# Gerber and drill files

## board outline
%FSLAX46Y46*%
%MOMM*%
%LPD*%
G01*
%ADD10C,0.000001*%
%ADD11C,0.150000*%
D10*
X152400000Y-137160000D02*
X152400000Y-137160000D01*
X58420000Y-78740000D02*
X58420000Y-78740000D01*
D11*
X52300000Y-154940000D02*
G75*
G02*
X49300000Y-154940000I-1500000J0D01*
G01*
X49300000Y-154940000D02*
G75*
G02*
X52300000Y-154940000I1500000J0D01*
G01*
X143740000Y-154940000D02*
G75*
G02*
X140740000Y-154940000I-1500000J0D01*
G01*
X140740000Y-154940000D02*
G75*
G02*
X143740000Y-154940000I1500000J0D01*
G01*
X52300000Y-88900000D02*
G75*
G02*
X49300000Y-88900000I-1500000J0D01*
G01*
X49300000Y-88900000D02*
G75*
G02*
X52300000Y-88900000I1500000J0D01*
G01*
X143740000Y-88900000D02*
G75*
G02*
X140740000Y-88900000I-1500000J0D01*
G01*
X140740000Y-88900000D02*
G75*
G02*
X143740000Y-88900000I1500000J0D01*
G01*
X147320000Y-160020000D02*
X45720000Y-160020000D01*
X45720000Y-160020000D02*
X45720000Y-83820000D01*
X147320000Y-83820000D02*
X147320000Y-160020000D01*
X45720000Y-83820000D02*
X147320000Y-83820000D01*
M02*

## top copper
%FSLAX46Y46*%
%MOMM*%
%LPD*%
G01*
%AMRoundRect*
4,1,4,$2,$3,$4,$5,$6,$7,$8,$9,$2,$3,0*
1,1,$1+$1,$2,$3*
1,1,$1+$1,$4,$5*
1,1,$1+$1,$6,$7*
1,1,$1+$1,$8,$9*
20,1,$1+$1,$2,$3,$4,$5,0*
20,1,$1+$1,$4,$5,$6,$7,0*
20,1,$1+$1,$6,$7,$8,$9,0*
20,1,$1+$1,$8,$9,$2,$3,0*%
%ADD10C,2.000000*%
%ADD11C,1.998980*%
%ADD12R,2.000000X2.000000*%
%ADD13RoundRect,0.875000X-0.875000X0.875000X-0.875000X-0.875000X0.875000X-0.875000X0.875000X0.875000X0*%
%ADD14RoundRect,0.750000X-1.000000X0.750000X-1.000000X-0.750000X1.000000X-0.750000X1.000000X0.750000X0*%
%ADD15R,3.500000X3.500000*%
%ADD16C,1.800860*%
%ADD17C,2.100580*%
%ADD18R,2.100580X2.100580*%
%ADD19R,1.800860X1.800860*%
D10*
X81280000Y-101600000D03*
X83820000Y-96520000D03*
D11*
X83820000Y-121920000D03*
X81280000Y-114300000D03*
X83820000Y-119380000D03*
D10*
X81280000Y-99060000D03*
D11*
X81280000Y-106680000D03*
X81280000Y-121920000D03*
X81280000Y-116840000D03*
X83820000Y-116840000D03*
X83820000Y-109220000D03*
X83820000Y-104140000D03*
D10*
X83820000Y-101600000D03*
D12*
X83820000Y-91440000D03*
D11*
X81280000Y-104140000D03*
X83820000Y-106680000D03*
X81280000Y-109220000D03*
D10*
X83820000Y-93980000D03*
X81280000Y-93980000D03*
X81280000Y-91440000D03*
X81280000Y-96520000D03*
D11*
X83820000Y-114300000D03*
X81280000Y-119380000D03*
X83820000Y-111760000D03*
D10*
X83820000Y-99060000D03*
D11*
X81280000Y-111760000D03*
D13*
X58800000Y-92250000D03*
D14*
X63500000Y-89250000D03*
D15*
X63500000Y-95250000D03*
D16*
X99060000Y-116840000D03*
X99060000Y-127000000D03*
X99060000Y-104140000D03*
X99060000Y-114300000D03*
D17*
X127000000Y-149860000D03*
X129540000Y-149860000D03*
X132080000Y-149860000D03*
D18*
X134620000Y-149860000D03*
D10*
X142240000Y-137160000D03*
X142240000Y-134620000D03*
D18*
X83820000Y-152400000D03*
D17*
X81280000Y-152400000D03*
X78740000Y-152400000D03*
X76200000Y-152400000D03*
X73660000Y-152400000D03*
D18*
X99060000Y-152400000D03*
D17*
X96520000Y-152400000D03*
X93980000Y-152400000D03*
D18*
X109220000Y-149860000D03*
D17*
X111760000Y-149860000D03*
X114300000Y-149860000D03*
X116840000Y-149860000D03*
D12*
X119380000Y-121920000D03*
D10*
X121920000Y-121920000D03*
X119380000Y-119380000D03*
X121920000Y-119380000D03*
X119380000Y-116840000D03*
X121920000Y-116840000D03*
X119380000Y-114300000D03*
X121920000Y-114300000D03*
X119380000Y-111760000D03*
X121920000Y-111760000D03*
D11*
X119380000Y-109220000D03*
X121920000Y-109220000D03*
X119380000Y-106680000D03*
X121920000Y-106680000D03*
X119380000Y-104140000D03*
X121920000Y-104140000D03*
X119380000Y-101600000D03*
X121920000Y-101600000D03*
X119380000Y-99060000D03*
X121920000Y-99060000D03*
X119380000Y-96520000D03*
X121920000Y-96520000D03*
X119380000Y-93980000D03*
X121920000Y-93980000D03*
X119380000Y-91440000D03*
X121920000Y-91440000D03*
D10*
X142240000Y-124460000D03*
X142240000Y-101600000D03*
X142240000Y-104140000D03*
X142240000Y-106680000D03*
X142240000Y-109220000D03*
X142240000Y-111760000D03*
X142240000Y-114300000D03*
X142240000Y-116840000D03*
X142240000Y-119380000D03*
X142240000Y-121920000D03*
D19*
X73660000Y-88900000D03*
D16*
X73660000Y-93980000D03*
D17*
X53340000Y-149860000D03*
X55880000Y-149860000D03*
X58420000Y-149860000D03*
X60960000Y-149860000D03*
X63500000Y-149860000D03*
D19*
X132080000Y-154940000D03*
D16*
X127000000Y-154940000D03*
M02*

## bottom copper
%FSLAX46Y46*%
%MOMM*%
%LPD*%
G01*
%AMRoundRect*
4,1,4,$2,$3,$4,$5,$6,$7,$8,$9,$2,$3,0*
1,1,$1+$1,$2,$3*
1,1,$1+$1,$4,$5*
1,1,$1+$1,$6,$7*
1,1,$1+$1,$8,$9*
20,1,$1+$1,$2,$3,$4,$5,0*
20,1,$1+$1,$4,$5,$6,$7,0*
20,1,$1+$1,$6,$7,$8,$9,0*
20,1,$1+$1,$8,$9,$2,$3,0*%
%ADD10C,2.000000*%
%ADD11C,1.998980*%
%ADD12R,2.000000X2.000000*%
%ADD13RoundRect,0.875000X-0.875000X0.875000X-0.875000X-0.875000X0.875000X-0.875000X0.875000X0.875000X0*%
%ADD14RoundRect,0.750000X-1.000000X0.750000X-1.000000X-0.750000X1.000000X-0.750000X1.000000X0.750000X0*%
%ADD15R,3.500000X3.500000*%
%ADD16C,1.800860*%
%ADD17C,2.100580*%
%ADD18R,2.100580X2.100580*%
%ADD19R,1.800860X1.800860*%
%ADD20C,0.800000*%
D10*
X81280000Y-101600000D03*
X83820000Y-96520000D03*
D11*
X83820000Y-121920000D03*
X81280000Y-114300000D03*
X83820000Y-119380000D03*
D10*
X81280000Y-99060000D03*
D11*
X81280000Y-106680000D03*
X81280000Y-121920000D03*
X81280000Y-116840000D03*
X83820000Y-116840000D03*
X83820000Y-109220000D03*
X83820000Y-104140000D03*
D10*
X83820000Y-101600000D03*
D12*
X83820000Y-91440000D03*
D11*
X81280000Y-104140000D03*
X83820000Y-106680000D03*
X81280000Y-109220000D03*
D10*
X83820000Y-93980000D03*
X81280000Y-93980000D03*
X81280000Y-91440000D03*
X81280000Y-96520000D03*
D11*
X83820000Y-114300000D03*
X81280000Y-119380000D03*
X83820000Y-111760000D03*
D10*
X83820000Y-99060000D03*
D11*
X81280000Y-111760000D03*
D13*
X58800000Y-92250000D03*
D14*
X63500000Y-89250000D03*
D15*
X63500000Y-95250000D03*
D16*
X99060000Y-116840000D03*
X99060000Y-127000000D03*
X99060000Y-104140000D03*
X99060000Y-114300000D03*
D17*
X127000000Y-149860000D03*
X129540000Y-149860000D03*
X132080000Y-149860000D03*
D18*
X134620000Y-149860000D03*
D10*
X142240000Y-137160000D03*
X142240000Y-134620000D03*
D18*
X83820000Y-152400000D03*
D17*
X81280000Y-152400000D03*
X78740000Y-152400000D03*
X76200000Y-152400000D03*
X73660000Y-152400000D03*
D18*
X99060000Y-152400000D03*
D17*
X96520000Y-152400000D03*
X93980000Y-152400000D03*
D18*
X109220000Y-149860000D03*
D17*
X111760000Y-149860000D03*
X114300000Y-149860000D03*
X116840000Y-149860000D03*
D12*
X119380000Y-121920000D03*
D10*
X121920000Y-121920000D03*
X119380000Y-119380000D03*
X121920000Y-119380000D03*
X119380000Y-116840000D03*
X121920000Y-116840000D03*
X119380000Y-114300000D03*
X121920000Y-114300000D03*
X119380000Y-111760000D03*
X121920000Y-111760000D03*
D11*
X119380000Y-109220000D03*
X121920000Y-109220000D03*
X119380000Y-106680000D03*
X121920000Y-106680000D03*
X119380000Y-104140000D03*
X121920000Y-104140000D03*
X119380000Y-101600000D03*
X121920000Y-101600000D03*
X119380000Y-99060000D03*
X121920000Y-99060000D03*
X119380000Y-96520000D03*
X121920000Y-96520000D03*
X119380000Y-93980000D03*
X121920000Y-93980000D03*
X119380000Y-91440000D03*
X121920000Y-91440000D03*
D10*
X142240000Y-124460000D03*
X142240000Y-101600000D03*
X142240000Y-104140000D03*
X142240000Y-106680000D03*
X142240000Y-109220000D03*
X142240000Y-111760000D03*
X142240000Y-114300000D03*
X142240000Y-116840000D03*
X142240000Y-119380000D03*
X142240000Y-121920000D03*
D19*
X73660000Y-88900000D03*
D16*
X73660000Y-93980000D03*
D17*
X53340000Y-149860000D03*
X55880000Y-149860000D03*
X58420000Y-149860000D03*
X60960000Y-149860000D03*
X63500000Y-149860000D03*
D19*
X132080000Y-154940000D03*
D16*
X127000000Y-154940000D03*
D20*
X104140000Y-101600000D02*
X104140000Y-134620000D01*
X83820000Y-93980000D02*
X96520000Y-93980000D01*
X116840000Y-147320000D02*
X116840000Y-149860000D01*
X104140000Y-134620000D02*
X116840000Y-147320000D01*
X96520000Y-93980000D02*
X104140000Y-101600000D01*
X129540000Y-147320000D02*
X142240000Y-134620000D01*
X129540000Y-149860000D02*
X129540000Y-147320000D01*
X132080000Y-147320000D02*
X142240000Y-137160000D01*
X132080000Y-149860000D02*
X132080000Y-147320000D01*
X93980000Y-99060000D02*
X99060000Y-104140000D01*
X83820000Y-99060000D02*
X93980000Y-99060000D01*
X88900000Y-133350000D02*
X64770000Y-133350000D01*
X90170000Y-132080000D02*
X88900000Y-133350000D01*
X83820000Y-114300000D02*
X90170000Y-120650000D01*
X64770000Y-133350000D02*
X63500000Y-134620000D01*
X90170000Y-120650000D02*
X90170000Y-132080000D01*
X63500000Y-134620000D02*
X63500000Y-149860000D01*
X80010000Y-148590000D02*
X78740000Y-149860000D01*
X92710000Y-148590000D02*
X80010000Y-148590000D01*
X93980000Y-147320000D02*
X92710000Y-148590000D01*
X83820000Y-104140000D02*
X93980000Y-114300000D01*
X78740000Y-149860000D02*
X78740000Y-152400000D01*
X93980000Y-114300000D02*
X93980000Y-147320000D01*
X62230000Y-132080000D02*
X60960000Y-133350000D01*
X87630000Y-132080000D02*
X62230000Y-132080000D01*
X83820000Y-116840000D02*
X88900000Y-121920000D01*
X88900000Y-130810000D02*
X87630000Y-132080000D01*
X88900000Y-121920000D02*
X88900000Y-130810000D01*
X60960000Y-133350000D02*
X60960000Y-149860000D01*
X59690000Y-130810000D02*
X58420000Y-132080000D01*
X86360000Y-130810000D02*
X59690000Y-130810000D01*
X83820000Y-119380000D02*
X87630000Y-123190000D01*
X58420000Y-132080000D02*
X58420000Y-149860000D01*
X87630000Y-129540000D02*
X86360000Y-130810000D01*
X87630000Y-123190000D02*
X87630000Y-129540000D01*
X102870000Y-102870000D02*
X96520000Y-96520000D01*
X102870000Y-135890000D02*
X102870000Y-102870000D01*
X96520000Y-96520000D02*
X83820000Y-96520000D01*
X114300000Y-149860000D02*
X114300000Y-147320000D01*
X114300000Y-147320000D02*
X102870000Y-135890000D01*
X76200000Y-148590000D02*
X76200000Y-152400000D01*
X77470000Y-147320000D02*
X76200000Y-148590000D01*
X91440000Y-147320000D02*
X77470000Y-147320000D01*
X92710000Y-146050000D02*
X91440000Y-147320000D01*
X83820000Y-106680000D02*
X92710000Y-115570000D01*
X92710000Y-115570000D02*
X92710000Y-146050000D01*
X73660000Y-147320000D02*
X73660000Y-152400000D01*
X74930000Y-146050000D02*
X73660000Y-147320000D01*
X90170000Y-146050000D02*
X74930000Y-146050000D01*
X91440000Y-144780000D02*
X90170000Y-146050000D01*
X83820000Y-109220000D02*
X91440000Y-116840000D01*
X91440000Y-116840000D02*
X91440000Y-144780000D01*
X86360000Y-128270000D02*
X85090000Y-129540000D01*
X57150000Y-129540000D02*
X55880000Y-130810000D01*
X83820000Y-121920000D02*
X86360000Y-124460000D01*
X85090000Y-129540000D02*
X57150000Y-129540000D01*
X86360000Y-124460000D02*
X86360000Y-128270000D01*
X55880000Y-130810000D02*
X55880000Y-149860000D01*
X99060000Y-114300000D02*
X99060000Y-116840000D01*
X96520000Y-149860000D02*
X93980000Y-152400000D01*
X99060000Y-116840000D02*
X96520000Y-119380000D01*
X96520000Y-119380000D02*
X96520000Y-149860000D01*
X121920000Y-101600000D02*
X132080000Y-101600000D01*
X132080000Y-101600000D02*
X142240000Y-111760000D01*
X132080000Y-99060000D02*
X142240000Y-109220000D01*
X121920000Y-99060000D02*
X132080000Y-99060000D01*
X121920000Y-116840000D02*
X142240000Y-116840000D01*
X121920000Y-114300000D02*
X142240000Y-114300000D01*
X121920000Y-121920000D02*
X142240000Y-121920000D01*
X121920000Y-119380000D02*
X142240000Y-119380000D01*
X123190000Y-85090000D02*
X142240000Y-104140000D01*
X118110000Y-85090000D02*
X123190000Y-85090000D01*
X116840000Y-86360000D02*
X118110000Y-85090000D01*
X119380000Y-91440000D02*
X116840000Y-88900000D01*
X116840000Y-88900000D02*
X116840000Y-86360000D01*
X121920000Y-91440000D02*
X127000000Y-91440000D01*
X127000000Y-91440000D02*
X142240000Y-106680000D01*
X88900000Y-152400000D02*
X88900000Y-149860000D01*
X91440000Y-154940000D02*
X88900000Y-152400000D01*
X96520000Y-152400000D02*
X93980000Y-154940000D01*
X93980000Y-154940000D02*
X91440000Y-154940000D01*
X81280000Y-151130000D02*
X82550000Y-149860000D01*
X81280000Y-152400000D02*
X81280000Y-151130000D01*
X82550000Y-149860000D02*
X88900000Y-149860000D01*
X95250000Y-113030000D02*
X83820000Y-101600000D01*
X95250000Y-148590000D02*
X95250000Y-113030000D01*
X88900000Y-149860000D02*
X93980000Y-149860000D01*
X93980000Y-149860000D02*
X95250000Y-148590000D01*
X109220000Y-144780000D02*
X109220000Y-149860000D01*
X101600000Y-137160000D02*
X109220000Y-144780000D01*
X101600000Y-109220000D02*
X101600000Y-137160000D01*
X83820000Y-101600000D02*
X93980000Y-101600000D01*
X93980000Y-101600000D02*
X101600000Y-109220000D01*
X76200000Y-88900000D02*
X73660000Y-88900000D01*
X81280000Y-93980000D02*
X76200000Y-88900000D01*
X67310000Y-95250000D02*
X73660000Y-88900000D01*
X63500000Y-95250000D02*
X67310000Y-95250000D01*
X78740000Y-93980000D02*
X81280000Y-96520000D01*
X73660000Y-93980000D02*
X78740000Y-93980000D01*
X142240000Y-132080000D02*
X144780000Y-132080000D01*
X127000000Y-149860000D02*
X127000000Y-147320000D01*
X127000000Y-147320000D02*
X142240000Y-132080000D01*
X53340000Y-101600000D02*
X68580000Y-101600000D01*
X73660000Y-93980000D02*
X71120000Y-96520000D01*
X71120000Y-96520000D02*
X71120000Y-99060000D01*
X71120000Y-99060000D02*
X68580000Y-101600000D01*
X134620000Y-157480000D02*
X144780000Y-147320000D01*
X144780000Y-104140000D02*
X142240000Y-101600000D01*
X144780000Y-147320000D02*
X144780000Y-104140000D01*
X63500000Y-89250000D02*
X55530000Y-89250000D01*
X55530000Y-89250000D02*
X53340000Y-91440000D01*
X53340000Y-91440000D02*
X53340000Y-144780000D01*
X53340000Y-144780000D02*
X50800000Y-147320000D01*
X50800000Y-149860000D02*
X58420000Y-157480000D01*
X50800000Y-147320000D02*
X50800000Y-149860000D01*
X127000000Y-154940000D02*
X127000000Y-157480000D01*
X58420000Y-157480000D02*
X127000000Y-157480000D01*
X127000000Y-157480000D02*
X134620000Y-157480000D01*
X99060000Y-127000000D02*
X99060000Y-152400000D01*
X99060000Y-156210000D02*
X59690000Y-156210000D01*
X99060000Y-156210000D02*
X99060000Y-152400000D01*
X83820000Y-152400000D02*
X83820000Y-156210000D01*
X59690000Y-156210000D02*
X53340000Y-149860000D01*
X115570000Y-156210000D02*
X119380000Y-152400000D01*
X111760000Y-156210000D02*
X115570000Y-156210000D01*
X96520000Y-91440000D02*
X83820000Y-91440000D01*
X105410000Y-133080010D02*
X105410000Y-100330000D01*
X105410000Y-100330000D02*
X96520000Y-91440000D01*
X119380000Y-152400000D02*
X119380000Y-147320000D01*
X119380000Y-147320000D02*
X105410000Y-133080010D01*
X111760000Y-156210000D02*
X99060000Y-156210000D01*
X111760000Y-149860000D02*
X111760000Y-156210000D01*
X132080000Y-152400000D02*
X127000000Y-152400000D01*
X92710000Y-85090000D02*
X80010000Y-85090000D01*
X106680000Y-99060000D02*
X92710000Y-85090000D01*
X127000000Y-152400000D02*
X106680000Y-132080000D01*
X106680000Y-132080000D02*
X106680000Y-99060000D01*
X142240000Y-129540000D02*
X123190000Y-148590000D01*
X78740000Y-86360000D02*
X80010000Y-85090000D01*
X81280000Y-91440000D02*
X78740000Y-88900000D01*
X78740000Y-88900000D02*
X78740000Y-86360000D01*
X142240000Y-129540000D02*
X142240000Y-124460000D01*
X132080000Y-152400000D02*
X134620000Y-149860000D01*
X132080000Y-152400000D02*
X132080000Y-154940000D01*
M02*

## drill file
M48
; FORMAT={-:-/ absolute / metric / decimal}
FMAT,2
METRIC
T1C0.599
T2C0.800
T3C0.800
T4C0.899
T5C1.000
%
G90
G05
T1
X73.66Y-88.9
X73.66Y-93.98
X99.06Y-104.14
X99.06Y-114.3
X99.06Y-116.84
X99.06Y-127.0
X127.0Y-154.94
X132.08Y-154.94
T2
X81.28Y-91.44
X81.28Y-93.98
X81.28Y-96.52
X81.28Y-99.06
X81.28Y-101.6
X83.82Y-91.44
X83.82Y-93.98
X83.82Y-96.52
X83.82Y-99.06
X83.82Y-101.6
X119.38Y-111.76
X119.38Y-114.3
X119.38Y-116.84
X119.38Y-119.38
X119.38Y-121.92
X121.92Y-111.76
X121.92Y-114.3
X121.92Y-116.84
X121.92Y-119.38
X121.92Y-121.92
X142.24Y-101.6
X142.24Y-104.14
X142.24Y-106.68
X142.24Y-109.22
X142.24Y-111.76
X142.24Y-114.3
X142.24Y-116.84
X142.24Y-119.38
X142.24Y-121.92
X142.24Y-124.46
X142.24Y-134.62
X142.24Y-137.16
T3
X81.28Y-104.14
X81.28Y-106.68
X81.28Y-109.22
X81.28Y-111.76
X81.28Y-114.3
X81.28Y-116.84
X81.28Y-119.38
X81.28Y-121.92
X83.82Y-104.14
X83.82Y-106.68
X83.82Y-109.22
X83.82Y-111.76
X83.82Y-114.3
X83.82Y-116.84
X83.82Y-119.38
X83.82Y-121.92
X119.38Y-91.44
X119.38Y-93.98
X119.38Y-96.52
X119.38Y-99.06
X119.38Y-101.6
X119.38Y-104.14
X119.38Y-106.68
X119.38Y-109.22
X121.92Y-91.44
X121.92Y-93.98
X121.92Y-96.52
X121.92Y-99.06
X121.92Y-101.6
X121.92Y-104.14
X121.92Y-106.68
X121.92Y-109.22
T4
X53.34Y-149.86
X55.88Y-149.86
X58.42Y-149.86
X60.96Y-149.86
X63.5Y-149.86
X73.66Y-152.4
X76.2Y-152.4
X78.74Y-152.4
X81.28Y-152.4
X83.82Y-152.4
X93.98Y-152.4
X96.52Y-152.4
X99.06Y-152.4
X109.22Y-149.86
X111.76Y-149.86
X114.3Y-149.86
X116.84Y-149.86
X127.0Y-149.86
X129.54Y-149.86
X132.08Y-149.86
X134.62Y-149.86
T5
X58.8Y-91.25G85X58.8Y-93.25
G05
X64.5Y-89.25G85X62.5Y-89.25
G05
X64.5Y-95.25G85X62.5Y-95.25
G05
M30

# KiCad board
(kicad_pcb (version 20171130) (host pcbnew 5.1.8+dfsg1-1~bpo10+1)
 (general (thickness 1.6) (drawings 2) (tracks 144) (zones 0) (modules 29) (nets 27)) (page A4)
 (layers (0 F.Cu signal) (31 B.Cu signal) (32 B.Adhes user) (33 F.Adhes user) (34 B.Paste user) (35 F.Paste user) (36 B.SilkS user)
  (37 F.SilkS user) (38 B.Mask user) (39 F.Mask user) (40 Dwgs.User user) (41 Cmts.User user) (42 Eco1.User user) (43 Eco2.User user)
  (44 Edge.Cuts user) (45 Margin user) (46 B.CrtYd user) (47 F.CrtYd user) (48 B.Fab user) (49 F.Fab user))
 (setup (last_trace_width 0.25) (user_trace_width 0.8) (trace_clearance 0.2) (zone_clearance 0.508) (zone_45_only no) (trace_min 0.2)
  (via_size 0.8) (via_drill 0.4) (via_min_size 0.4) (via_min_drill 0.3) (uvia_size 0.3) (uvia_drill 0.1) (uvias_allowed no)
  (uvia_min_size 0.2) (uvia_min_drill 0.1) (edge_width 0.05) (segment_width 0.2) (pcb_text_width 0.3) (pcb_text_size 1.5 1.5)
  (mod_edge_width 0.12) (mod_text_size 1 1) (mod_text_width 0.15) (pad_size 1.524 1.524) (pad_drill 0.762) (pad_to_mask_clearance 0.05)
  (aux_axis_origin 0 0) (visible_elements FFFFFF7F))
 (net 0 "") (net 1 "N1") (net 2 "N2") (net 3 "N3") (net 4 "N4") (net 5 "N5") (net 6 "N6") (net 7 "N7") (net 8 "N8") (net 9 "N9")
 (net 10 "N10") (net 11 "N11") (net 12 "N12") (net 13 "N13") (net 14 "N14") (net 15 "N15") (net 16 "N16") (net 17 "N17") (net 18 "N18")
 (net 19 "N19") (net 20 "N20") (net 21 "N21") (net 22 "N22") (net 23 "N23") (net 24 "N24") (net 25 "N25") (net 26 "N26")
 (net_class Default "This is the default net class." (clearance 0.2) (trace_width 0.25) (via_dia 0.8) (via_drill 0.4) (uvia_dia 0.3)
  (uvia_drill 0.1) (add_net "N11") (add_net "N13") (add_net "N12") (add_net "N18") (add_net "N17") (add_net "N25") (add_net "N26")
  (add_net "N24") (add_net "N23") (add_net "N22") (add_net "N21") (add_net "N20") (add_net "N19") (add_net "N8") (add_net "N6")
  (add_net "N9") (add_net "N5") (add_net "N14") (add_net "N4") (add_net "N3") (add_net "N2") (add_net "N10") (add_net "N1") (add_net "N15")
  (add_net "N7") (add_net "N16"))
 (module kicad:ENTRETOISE (layer F.Cu) (at 50.8 154.94)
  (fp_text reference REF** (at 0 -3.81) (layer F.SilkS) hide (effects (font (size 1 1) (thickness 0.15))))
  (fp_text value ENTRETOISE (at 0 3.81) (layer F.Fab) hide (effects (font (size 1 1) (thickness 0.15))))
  (fp_circle (center 0 0) (end 1.5 0) (layer Edge.Cuts) (width 0.15)))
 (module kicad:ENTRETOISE (layer F.Cu) (at 142.24 154.94)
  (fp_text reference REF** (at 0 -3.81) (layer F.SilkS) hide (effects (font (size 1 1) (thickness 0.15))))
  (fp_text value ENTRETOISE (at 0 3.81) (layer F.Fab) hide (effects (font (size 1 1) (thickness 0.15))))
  (fp_circle (center 0 0) (end 1.5 0) (layer Edge.Cuts) (width 0.15)))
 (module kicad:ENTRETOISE (layer F.Cu) (at 50.8 88.9)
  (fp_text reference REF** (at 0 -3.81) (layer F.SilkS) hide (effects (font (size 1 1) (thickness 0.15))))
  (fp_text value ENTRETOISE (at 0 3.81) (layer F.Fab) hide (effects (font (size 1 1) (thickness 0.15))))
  (fp_circle (center 0 0) (end 1.5 0) (layer Edge.Cuts) (width 0.15)))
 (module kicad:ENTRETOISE (layer F.Cu) (at 142.24 88.9)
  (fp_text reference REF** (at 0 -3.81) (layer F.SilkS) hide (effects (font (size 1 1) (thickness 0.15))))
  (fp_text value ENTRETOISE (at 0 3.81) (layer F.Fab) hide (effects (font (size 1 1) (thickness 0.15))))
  (fp_circle (center 0 0) (end 1.5 0) (layer Edge.Cuts) (width 0.15)))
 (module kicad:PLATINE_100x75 (layer F.Cu) (at 96.52 121.92)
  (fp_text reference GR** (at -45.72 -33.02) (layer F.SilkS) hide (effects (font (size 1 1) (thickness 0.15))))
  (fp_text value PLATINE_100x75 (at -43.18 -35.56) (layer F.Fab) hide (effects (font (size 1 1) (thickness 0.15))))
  (fp_line (start 50.8 38.1) (end -50.8 38.1) (layer Edge.Cuts) (width 0.15))
  (fp_line (start -50.8 38.1) (end -50.8 -38.1) (layer Edge.Cuts) (width 0.15))
  (fp_line (start 50.8 -38.1) (end 50.8 38.1) (layer Edge.Cuts) (width 0.15))
  (fp_line (start -50.8 -38.1) (end 50.8 -38.1) (layer Edge.Cuts) (width 0.15)))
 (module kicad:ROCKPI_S (layer F.Cu) (at 101.6 106.68)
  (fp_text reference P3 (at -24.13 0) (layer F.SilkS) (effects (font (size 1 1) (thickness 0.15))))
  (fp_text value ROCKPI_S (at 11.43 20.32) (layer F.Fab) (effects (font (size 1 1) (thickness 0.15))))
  (pad 10 thru_hole circle (at -20.32 -5.08 270) (size 2 2) (drill 0.8) (layers *.Cu *.Mask F.SilkS))
  (pad 5 thru_hole circle (at -17.78 -10.16 270) (size 2 2) (drill 0.8) (layers *.Cu *.Mask F.SilkS) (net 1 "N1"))
  (pad 25 thru_hole circle (at -17.78 15.24 270) (size 1.99898 1.99898) (drill 0.8001) (layers *.Cu *.Mask F.SilkS) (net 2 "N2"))
  (pad 20 thru_hole circle (at -20.32 7.62 270) (size 1.99898 1.99898) (drill 0.8001) (layers *.Cu *.Mask F.SilkS))
  (pad 23 thru_hole circle (at -17.78 12.7 270) (size 1.99898 1.99898) (drill 0.8001) (layers *.Cu *.Mask F.SilkS) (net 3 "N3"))
  (pad 8 thru_hole circle (at -20.32 -7.62 270) (size 2 2) (drill 0.8) (layers *.Cu *.Mask F.SilkS))
  (pad 14 thru_hole circle (at -20.32 0 270) (size 1.99898 1.99898) (drill 0.8001) (layers *.Cu *.Mask F.SilkS))
  (pad 26 thru_hole circle (at -20.32 15.24 270) (size 1.99898 1.99898) (drill 0.8001) (layers *.Cu *.Mask F.SilkS))
  (pad 22 thru_hole circle (at -20.32 10.16 270) (size 1.99898 1.99898) (drill 0.8001) (layers *.Cu *.Mask F.SilkS))
  (pad 21 thru_hole circle (at -17.78 10.16 270) (size 1.99898 1.99898) (drill 0.8001) (layers *.Cu *.Mask F.SilkS) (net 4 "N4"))
  (pad 15 thru_hole circle (at -17.78 2.54 270) (size 1.99898 1.99898) (drill 0.8001) (layers *.Cu *.Mask F.SilkS) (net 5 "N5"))
  (pad 11 thru_hole circle (at -17.78 -2.54 270) (size 1.99898 1.99898) (drill 0.8001) (layers *.Cu *.Mask F.SilkS) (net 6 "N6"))
  (pad 9 thru_hole circle (at -17.78 -5.08 270) (size 2 2) (drill 0.8) (layers *.Cu *.Mask F.SilkS) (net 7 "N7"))
  (pad 1 thru_hole rect (at -17.78 -15.24 270) (size 2 2) (drill 0.8) (layers *.Cu *.Mask F.SilkS) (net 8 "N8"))
  (pad 12 thru_hole circle (at -20.32 -2.54 270) (size 1.99898 1.99898) (drill 0.8001) (layers *.Cu *.Mask F.SilkS))
  (pad 13 thru_hole circle (at -17.78 0 270) (size 1.99898 1.99898) (drill 0.8001) (layers *.Cu *.Mask F.SilkS) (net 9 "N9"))
  (pad 16 thru_hole circle (at -20.32 2.54 270) (size 1.99898 1.99898) (drill 0.8001) (layers *.Cu *.Mask F.SilkS))
  (pad 3 thru_hole circle (at -17.78 -12.7 270) (size 2 2) (drill 0.8) (layers *.Cu *.Mask F.SilkS) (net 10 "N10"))
  (pad 4 thru_hole circle (at -20.32 -12.7 270) (size 2 2) (drill 0.8) (layers *.Cu *.Mask F.SilkS) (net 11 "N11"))
  (pad 2 thru_hole circle (at -20.32 -15.24 270) (size 2 2) (drill 0.8) (layers *.Cu *.Mask F.SilkS) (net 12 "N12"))
  (pad 6 thru_hole circle (at -20.32 -10.16 270) (size 2 2) (drill 0.8) (layers *.Cu *.Mask F.SilkS) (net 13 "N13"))
  (pad 19 thru_hole circle (at -17.78 7.62 270) (size 1.99898 1.99898) (drill 0.8001) (layers *.Cu *.Mask F.SilkS) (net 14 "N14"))
  (pad 24 thru_hole circle (at -20.32 12.7 270) (size 1.99898 1.99898) (drill 0.8001) (layers *.Cu *.Mask F.SilkS))
  (pad 17 thru_hole circle (at -17.78 5.08) (size 1.99898 1.99898) (drill 0.8001) (layers *.Cu *.Mask F.SilkS))
  (pad 7 thru_hole circle (at -17.78 -7.62 270) (size 2 2) (drill 0.8) (layers *.Cu *.Mask F.SilkS) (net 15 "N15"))
  (pad 18 thru_hole circle (at -20.32 5.08 270) (size 1.99898 1.99898) (drill 0.8001) (layers *.Cu *.Mask F.SilkS)))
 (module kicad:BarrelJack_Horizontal (layer F.Cu) (at 63.5 95.25 270)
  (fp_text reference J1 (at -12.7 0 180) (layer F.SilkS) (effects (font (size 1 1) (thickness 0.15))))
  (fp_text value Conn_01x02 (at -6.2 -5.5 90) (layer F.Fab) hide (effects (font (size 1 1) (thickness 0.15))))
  (pad 3 thru_hole roundrect (at -3 4.7 270) (size 3.5 3.5) (drill oval 3 1) (layers *.Cu *.Mask) (roundrect_rratio 0.25))
  (pad 2 thru_hole roundrect (at -6 0 270) (size 3 3.5) (drill oval 1 3) (layers *.Cu *.Mask) (roundrect_rratio 0.25) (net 13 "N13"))
  (pad 1 thru_hole rect (at 0 0 270) (size 3.5 3.5) (drill oval 1 3) (layers *.Cu *.Mask) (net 11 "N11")))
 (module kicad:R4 (layer F.Cu) (at 99.06 121.92 270) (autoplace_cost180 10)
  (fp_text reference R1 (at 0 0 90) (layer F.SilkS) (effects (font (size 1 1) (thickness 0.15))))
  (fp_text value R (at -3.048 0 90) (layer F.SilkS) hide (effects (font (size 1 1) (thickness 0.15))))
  (pad 1 thru_hole circle (at -5.08 0 270) (size 1.80086 1.80086) (drill 0.59944) (layers *.Cu *.Mask F.SilkS) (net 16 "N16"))
  (pad 2 thru_hole circle (at 5.08 0 270) (size 1.80086 1.80086) (drill 0.59944) (layers *.Cu *.Mask F.SilkS) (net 8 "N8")))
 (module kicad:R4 (layer F.Cu) (at 99.06 109.22 270) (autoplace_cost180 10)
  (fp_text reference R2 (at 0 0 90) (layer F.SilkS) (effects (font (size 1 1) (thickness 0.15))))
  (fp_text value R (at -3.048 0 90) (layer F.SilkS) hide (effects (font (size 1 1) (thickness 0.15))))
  (pad 1 thru_hole circle (at -5.08 0 270) (size 1.80086 1.80086) (drill 0.59944) (layers *.Cu *.Mask F.SilkS) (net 15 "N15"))
  (pad 2 thru_hole circle (at 5.08 0 270) (size 1.80086 1.80086) (drill 0.59944) (layers *.Cu *.Mask F.SilkS) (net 16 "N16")))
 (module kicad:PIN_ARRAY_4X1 (layer F.Cu) (at 130.81 149.86 180)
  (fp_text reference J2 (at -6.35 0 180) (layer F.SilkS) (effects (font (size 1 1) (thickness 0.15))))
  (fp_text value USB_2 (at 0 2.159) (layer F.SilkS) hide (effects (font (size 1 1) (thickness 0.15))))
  (pad 4 thru_hole circle (at 3.81 0 180) (size 2.10058 2.10058) (drill 0.89916) (layers *.Cu *.Mask F.SilkS) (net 13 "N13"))
  (pad 3 thru_hole circle (at 1.27 0 180) (size 2.10058 2.10058) (drill 0.89916) (layers *.Cu *.Mask F.SilkS) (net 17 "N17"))
  (pad 2 thru_hole circle (at -1.27 0 180) (size 2.10058 2.10058) (drill 0.89916) (layers *.Cu *.Mask F.SilkS) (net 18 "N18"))
  (pad 1 thru_hole rect (at -3.81 0 180) (size 2.10058 2.10058) (drill 0.89916) (layers *.Cu *.Mask F.SilkS) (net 12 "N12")))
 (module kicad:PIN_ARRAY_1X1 (layer F.Cu) (at 142.24 137.16)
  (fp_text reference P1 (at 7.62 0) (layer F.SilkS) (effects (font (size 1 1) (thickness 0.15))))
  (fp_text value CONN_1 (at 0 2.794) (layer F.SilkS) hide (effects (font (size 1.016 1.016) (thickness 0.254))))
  (pad 1 thru_hole circle (at 0 0) (size 2 2) (drill 0.8) (layers *.Cu *.Mask F.SilkS) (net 18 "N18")))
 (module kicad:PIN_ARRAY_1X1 (layer F.Cu) (at 142.24 134.62)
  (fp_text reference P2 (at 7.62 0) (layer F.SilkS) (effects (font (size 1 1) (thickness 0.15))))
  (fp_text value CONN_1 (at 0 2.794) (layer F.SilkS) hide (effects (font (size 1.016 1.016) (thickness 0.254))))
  (pad 1 thru_hole circle (at 0 0) (size 2 2) (drill 0.8) (layers *.Cu *.Mask F.SilkS) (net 17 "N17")))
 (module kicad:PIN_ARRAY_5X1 (layer F.Cu) (at 78.74 152.4 180)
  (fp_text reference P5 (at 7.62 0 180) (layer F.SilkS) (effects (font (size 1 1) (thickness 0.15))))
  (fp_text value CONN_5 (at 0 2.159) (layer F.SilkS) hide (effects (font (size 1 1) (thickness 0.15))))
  (pad 1 thru_hole rect (at -5.08 0 180) (size 2.10058 2.10058) (drill 0.89916) (layers *.Cu *.Mask F.SilkS) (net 8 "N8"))
  (pad 2 thru_hole circle (at -2.54 0 180) (size 2.10058 2.10058) (drill 0.89916) (layers *.Cu *.Mask F.SilkS) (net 7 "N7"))
  (pad 3 thru_hole circle (at 0 0 180) (size 2.10058 2.10058) (drill 0.89916) (layers *.Cu *.Mask F.SilkS) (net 6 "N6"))
  (pad 4 thru_hole circle (at 2.54 0 180) (size 2.10058 2.10058) (drill 0.89916) (layers *.Cu *.Mask F.SilkS) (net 9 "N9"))
  (pad 5 thru_hole circle (at 5.08 0 180) (size 2.10058 2.10058) (drill 0.89916) (layers *.Cu *.Mask F.SilkS) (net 5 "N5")))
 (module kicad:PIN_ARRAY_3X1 (layer F.Cu) (at 96.52 152.4 180)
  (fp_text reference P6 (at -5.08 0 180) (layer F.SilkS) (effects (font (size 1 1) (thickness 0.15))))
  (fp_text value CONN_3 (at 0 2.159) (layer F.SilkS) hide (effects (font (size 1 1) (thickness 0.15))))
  (pad 1 thru_hole rect (at -2.54 0 180) (size 2.10058 2.10058) (drill 0.89916) (layers *.Cu *.Mask F.SilkS) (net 8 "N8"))
  (pad 2 thru_hole circle (at 0 0 180) (size 2.10058 2.10058) (drill 0.89916) (layers *.Cu *.Mask F.SilkS) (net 7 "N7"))
  (pad 3 thru_hole circle (at 2.54 0 180) (size 2.10058 2.10058) (drill 0.89916) (layers *.Cu *.Mask F.SilkS) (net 16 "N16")))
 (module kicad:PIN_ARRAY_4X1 (layer F.Cu) (at 113.03 149.86)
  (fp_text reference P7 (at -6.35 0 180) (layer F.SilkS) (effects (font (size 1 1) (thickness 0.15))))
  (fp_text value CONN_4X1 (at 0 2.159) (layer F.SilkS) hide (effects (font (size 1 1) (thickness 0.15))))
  (pad 1 thru_hole rect (at -3.81 0) (size 2.10058 2.10058) (drill 0.89916) (layers *.Cu *.Mask F.SilkS) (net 7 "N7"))
  (pad 2 thru_hole circle (at -1.27 0) (size 2.10058 2.10058) (drill 0.89916) (layers *.Cu *.Mask F.SilkS) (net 8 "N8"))
  (pad 3 thru_hole circle (at 1.27 0) (size 2.10058 2.10058) (drill 0.89916) (layers *.Cu *.Mask F.SilkS) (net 1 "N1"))
  (pad 4 thru_hole circle (at 3.81 0) (size 2.10058 2.10058) (drill 0.89916) (layers *.Cu *.Mask F.SilkS) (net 10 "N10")))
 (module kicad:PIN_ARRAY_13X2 (layer F.Cu) (at 120.65 106.68 90)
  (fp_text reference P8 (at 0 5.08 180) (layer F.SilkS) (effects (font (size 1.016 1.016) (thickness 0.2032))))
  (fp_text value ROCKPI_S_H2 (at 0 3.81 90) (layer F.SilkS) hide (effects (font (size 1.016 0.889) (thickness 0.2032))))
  (pad 1 thru_hole rect (at -15.24 -1.27 90) (size 2 2) (drill 0.8) (layers *.Cu *.Mask F.SilkS))
  (pad 2 thru_hole circle (at -15.24 1.27 90) (size 2 2) (drill 0.8) (layers *.Cu *.Mask F.SilkS) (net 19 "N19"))
  (pad 3 thru_hole circle (at -12.7 -1.27 90) (size 2 2) (drill 0.8) (layers *.Cu *.Mask F.SilkS))
  (pad 4 thru_hole circle (at -12.7 1.27 90) (size 2 2) (drill 0.8) (layers *.Cu *.Mask F.SilkS) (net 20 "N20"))
  (pad 5 thru_hole circle (at -10.16 -1.27 90) (size 2 2) (drill 0.8) (layers *.Cu *.Mask F.SilkS))
  (pad 6 thru_hole circle (at -10.16 1.27 90) (size 2 2) (drill 0.8) (layers *.Cu *.Mask F.SilkS) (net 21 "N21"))
  (pad 7 thru_hole circle (at -7.62 -1.27 90) (size 2 2) (drill 0.8) (layers *.Cu *.Mask F.SilkS))
  (pad 8 thru_hole circle (at -7.62 1.27 90) (size 2 2) (drill 0.8) (layers *.Cu *.Mask F.SilkS) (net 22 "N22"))
  (pad 9 thru_hole circle (at -5.08 -1.27 90) (size 2 2) (drill 0.8) (layers *.Cu *.Mask F.SilkS))
  (pad 10 thru_hole circle (at -5.08 1.27 90) (size 2 2) (drill 0.8) (layers *.Cu *.Mask F.SilkS))
  (pad 11 thru_hole circle (at -2.54 -1.27 90) (size 1.99898 1.99898) (drill 0.8001) (layers *.Cu *.Mask F.SilkS))
  (pad 12 thru_hole circle (at -2.54 1.27 90) (size 1.99898 1.99898) (drill 0.8001) (layers *.Cu *.Mask F.SilkS))
  (pad 13 thru_hole circle (at 0 -1.27 90) (size 1.99898 1.99898) (drill 0.8001) (layers *.Cu *.Mask F.SilkS))
  (pad 14 thru_hole circle (at 0 1.27 90) (size 1.99898 1.99898) (drill 0.8001) (layers *.Cu *.Mask F.SilkS))
  (pad 15 thru_hole circle (at 2.54 -1.27 90) (size 1.99898 1.99898) (drill 0.8001) (layers *.Cu *.Mask F.SilkS))
  (pad 16 thru_hole circle (at 2.54 1.27 90) (size 1.99898 1.99898) (drill 0.8001) (layers *.Cu *.Mask F.SilkS))
  (pad 17 thru_hole circle (at 5.08 -1.27 90) (size 1.99898 1.99898) (drill 0.8001) (layers *.Cu *.Mask F.SilkS))
  (pad 18 thru_hole circle (at 5.08 1.27 90) (size 1.99898 1.99898) (drill 0.8001) (layers *.Cu *.Mask F.SilkS) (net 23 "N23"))
  (pad 19 thru_hole circle (at 7.62 -1.27 90) (size 1.99898 1.99898) (drill 0.8001) (layers *.Cu *.Mask F.SilkS))
  (pad 20 thru_hole circle (at 7.62 1.27 90) (size 1.99898 1.99898) (drill 0.8001) (layers *.Cu *.Mask F.SilkS) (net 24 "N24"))
  (pad 21 thru_hole circle (at 10.16 -1.27 90) (size 1.99898 1.99898) (drill 0.8001) (layers *.Cu *.Mask F.SilkS))
  (pad 22 thru_hole circle (at 10.16 1.27 90) (size 1.99898 1.99898) (drill 0.8001) (layers *.Cu *.Mask F.SilkS))
  (pad 23 thru_hole circle (at 12.7 -1.27 90) (size 1.99898 1.99898) (drill 0.8001) (layers *.Cu *.Mask F.SilkS))
  (pad 24 thru_hole circle (at 12.7 1.27 90) (size 1.99898 1.99898) (drill 0.8001) (layers *.Cu *.Mask F.SilkS))
  (pad 25 thru_hole circle (at 15.24 -1.27 90) (size 1.99898 1.99898) (drill 0.8001) (layers *.Cu *.Mask F.SilkS) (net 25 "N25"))
  (pad 26 thru_hole circle (at 15.24 1.27 90) (size 1.99898 1.99898) (drill 0.8001) (layers *.Cu *.Mask F.SilkS) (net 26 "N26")))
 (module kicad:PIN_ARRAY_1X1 (layer F.Cu) (at 142.24 124.46 90)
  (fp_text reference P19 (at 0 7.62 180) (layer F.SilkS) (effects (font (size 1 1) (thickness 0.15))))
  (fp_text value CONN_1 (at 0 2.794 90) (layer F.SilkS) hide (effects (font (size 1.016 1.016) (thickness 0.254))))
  (pad 1 thru_hole circle (at 0 0 90) (size 2 2) (drill 0.8) (layers *.Cu *.Mask F.SilkS) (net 12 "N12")))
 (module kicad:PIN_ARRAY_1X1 (layer F.Cu) (at 142.24 101.6 90)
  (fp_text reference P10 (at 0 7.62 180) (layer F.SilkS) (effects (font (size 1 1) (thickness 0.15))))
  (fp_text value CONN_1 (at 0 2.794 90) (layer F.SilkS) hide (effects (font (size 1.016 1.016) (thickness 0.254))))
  (pad 1 thru_hole circle (at 0 0 90) (size 2 2) (drill 0.8) (layers *.Cu *.Mask F.SilkS) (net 13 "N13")))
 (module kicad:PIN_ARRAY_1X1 (layer F.Cu) (at 142.24 104.14 90)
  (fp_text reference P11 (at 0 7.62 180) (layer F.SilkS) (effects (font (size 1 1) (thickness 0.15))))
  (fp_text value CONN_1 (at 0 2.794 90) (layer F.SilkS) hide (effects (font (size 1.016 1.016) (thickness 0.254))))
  (pad 1 thru_hole circle (at 0 0 90) (size 2 2) (drill 0.8) (layers *.Cu *.Mask F.SilkS) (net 25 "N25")))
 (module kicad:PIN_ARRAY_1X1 (layer F.Cu) (at 142.24 106.68)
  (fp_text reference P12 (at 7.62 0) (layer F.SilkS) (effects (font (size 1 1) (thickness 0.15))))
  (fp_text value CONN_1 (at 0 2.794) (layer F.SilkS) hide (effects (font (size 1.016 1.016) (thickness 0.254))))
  (pad 1 thru_hole circle (at 0 0) (size 2 2) (drill 0.8) (layers *.Cu *.Mask F.SilkS) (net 26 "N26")))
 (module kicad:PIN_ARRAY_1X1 (layer F.Cu) (at 142.24 109.22)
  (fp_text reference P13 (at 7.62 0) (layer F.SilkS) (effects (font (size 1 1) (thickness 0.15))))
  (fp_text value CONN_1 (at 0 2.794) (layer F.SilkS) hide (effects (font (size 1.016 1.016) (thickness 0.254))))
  (pad 1 thru_hole circle (at 0 0) (size 2 2) (drill 0.8) (layers *.Cu *.Mask F.SilkS) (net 24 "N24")))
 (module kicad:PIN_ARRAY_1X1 (layer F.Cu) (at 142.24 111.76)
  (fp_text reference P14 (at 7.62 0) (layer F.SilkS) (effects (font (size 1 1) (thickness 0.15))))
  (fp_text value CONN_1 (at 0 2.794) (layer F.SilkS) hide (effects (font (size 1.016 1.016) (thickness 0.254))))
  (pad 1 thru_hole circle (at 0 0) (size 2 2) (drill 0.8) (layers *.Cu *.Mask F.SilkS) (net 23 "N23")))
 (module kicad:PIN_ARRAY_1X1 (layer F.Cu) (at 142.24 114.3)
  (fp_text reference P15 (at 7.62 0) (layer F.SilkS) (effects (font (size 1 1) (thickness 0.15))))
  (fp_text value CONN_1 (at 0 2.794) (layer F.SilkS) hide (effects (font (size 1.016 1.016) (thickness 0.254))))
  (pad 1 thru_hole circle (at 0 0) (size 2 2) (drill 0.8) (layers *.Cu *.Mask F.SilkS) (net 22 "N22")))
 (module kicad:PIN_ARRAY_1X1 (layer F.Cu) (at 142.24 116.84)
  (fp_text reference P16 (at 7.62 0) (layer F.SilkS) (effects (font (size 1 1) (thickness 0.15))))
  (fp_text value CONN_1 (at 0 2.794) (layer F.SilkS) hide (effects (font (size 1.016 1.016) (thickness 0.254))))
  (pad 1 thru_hole circle (at 0 0) (size 2 2) (drill 0.8) (layers *.Cu *.Mask F.SilkS) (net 21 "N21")))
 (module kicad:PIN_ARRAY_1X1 (layer F.Cu) (at 142.24 119.38)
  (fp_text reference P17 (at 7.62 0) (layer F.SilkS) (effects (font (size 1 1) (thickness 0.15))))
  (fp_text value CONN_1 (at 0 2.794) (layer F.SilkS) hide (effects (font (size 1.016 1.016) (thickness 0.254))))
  (pad 1 thru_hole circle (at 0 0) (size 2 2) (drill 0.8) (layers *.Cu *.Mask F.SilkS) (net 20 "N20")))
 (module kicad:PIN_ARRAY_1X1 (layer F.Cu) (at 142.24 121.92)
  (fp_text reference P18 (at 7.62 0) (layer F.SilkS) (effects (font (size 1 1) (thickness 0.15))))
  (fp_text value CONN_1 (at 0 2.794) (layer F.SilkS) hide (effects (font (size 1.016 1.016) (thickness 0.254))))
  (pad 1 thru_hole circle (at 0 0) (size 2 2) (drill 0.8) (layers *.Cu *.Mask F.SilkS) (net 19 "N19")))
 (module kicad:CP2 (layer F.Cu) (at 73.66 91.44 180)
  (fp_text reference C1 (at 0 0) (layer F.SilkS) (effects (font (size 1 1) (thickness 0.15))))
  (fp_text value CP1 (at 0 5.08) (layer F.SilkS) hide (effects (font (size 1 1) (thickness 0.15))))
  (pad 1 thru_hole rect (at 0 2.54 180) (size 1.80086 1.80086) (drill 0.59944) (layers *.Cu *.Mask F.SilkS) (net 11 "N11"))
  (pad 2 thru_hole circle (at 0 -2.54 180) (size 1.80086 1.80086) (drill 0.59944) (layers *.Cu *.Mask F.SilkS) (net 13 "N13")))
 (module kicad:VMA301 (layer F.Cu) (at 58.42 149.86)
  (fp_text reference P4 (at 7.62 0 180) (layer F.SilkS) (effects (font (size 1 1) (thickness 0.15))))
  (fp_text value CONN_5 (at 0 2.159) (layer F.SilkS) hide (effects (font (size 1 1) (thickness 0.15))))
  (pad 1 thru_hole circle (at -5.08 0) (size 2.10058 2.10058) (drill 0.89916) (layers *.Cu *.Mask F.SilkS) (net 8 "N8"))
  (pad 2 thru_hole circle (at -2.54 0) (size 2.10058 2.10058) (drill 0.89916) (layers *.Cu *.Mask F.SilkS) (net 2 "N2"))
  (pad 3 thru_hole circle (at 0 0) (size 2.10058 2.10058) (drill 0.89916) (layers *.Cu *.Mask F.SilkS) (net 3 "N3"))
  (pad 4 thru_hole circle (at 2.54 0) (size 2.10058 2.10058) (drill 0.89916) (layers *.Cu *.Mask F.SilkS) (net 4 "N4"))
  (pad 5 thru_hole circle (at 5.08 0) (size 2.10058 2.10058) (drill 0.89916) (layers *.Cu *.Mask F.SilkS) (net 14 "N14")))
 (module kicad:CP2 (layer F.Cu) (at 129.54 154.94 90)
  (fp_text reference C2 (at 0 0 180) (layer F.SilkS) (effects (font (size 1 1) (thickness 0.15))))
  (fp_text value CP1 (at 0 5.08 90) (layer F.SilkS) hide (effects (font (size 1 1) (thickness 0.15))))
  (pad 1 thru_hole rect (at 0 2.54 90) (size 1.80086 1.80086) (drill 0.59944) (layers *.Cu *.Mask F.SilkS) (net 12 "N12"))
  (pad 2 thru_hole circle (at 0 -2.54 90) (size 1.80086 1.80086) (drill 0.59944) (layers *.Cu *.Mask F.SilkS) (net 13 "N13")))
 (gr_line (start 152.4 137.16) (end 152.4 137.16) (layer Edge.Cuts) (width 0.000001))
 (gr_line (start 58.42 78.74) (end 58.42 78.74) (layer Edge.Cuts) (width 0.000001))
 (segment (start 104.14 101.6) (end 104.14 134.62) (width 0.8) (layer B.Cu) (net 10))
 (segment (start 83.82 93.98) (end 96.52 93.98) (width 0.8) (layer B.Cu) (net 10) (status 10))
 (segment (start 116.84 147.32) (end 116.84 149.86) (width 0.8) (layer B.Cu) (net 10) (status 20))
 (segment (start 104.14 134.62) (end 116.84 147.32) (width 0.8) (layer B.Cu) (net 10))
 (segment (start 96.52 93.98) (end 104.14 101.6) (width 0.8) (layer B.Cu) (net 10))
 (segment (start 129.54 147.32) (end 142.24 134.62) (width 0.8) (layer B.Cu) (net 17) (status 20))
 (segment (start 129.54 149.86) (end 129.54 147.32) (width 0.8) (layer B.Cu) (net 17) (status 10))
 (segment (start 132.08 147.32) (end 142.24 137.16) (width 0.8) (layer B.Cu) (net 18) (status 20))
 (segment (start 132.08 149.86) (end 132.08 147.32) (width 0.8) (layer B.Cu) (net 18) (status 10))
 (segment (start 93.98 99.06) (end 99.06 104.14) (width 0.8) (layer B.Cu) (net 15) (status 20))
 (segment (start 83.82 99.06) (end 93.98 99.06) (width 0.8) (layer B.Cu) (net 15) (status 10))
 (segment (start 88.9 133.35) (end 64.77 133.35) (width 0.8) (layer B.Cu) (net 14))
 (segment (start 90.17 132.08) (end 88.9 133.35) (width 0.8) (layer B.Cu) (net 14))
 (segment (start 83.82 114.3) (end 90.17 120.65) (width 0.8) (layer B.Cu) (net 14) (status 10))
 (segment (start 64.77 133.35) (end 63.5 134.62) (width 0.8) (layer B.Cu) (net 14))
 (segment (start 90.17 120.65) (end 90.17 132.08) (width 0.8) (layer B.Cu) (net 14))
 (segment (start 63.5 134.62) (end 63.5 149.86) (width 0.8) (layer B.Cu) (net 14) (status 20))
 (segment (start 80.01 148.59) (end 78.74 149.86) (width 0.8) (layer B.Cu) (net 6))
 (segment (start 92.71 148.59) (end 80.01 148.59) (width 0.8) (layer B.Cu) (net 6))
 (segment (start 93.98 147.32) (end 92.71 148.59) (width 0.8) (layer B.Cu) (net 6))
 (segment (start 83.82 104.14) (end 93.98 114.3) (width 0.8) (layer B.Cu) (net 6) (status 10))
 (segment (start 78.74 149.86) (end 78.74 152.4) (width 0.8) (layer B.Cu) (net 6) (status 20))
 (segment (start 93.98 114.3) (end 93.98 147.32) (width 0.8) (layer B.Cu) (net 6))
 (segment (start 62.23 132.08) (end 60.96 133.35) (width 0.8) (layer B.Cu) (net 4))
 (segment (start 87.63 132.08) (end 62.23 132.08) (width 0.8) (layer B.Cu) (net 4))
 (segment (start 83.82 116.84) (end 88.9 121.92) (width 0.8) (layer B.Cu) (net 4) (status 10))
 (segment (start 88.9 130.81) (end 87.63 132.08) (width 0.8) (layer B.Cu) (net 4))
 (segment (start 88.9 121.92) (end 88.9 130.81) (width 0.8) (layer B.Cu) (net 4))
 (segment (start 60.96 133.35) (end 60.96 149.86) (width 0.8) (layer B.Cu) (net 4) (status 20))
 (segment (start 59.69 130.81) (end 58.42 132.08) (width 0.8) (layer B.Cu) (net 3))
 (segment (start 86.36 130.81) (end 59.69 130.81) (width 0.8) (layer B.Cu) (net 3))
 (segment (start 83.82 119.38) (end 87.63 123.19) (width 0.8) (layer B.Cu) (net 3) (status 10))
 (segment (start 58.42 132.08) (end 58.42 149.86) (width 0.8) (layer B.Cu) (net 3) (status 20))
 (segment (start 87.63 129.54) (end 86.36 130.81) (width 0.8) (layer B.Cu) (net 3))
 (segment (start 87.63 123.19) (end 87.63 129.54) (width 0.8) (layer B.Cu) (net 3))
 (segment (start 102.87 102.87) (end 96.52 96.52) (width 0.8) (layer B.Cu) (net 1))
 (segment (start 102.87 135.89) (end 102.87 102.87) (width 0.8) (layer B.Cu) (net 1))
 (segment (start 96.52 96.52) (end 83.82 96.52) (width 0.8) (layer B.Cu) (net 1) (status 20))
 (segment (start 114.3 149.86) (end 114.3 147.32) (width 0.8) (layer B.Cu) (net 1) (status 10))
 (segment (start 114.3 147.32) (end 102.87 135.89) (width 0.8) (layer B.Cu) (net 1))
 (segment (start 76.2 148.59) (end 76.2 152.4) (width 0.8) (layer B.Cu) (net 9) (status 20))
 (segment (start 77.47 147.32) (end 76.2 148.59) (width 0.8) (layer B.Cu) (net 9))
 (segment (start 91.44 147.32) (end 77.47 147.32) (width 0.8) (layer B.Cu) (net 9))
 (segment (start 92.71 146.05) (end 91.44 147.32) (width 0.8) (layer B.Cu) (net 9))
 (segment (start 83.82 106.68) (end 92.71 115.57) (width 0.8) (layer B.Cu) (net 9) (status 10))
 (segment (start 92.71 115.57) (end 92.71 146.05) (width 0.8) (layer B.Cu) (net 9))
 (segment (start 73.66 147.32) (end 73.66 152.4) (width 0.8) (layer B.Cu) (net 5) (status 20))
 (segment (start 74.93 146.05) (end 73.66 147.32) (width 0.8) (layer B.Cu) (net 5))
 (segment (start 90.17 146.05) (end 74.93 146.05) (width 0.8) (layer B.Cu) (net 5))
 (segment (start 91.44 144.78) (end 90.17 146.05) (width 0.8) (layer B.Cu) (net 5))
 (segment (start 83.82 109.22) (end 91.44 116.84) (width 0.8) (layer B.Cu) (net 5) (status 10))
 (segment (start 91.44 116.84) (end 91.44 144.78) (width 0.8) (layer B.Cu) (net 5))
 (segment (start 86.36 128.27) (end 85.09 129.54) (width 0.8) (layer B.Cu) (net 2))
 (segment (start 57.15 129.54) (end 55.88 130.81) (width 0.8) (layer B.Cu) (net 2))
 (segment (start 83.82 121.92) (end 86.36 124.46) (width 0.8) (layer B.Cu) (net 2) (status 10))
 (segment (start 85.09 129.54) (end 57.15 129.54) (width 0.8) (layer B.Cu) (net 2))
 (segment (start 86.36 124.46) (end 86.36 128.27) (width 0.8) (layer B.Cu) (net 2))
 (segment (start 55.88 130.81) (end 55.88 149.86) (width 0.8) (layer B.Cu) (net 2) (status 20))
 (segment (start 99.06 114.3) (end 99.06 116.84) (width 0.8) (layer B.Cu) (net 16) (status 30))
 (segment (start 96.52 149.86) (end 93.98 152.4) (width 0.8) (layer B.Cu) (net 16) (status 20))
 (segment (start 99.06 116.84) (end 96.52 119.38) (width 0.8) (layer B.Cu) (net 16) (status 10))
 (segment (start 96.52 119.38) (end 96.52 149.86) (width 0.8) (layer B.Cu) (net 16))
 (segment (start 121.92 101.6) (end 132.08 101.6) (width 0.8) (layer B.Cu) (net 23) (status 10))
 (segment (start 132.08 101.6) (end 142.24 111.76) (width 0.8) (layer B.Cu) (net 23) (status 20))
 (segment (start 132.08 99.06) (end 142.24 109.22) (width 0.8) (layer B.Cu) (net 24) (status 20))
 (segment (start 121.92 99.06) (end 132.08 99.06) (width 0.8) (layer B.Cu) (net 24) (status 10))
 (segment (start 121.92 116.84) (end 142.24 116.84) (width 0.8) (layer B.Cu) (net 21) (status 30))
 (segment (start 121.92 114.3) (end 142.24 114.3) (width 0.8) (layer B.Cu) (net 22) (status 30))
 (segment (start 121.92 121.92) (end 142.24 121.92) (width 0.8) (layer B.Cu) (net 19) (status 30))
 (segment (start 121.92 119.38) (end 142.24 119.38) (width 0.8) (layer B.Cu) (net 20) (status 30))
 (segment (start 123.19 85.09) (end 142.24 104.14) (width 0.8) (layer B.Cu) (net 25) (status 20))
 (segment (start 118.11 85.09) (end 123.19 85.09) (width 0.8) (layer B.Cu) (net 25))
 (segment (start 116.84 86.36) (end 118.11 85.09) (width 0.8) (layer B.Cu) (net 25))
 (segment (start 119.38 91.44) (end 116.84 88.9) (width 0.8) (layer B.Cu) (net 25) (status 10))
 (segment (start 116.84 88.9) (end 116.84 86.36) (width 0.8) (layer B.Cu) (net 25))
 (segment (start 121.92 91.44) (end 127 91.44) (width 0.8) (layer B.Cu) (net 26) (status 10))
 (segment (start 127 91.44) (end 142.24 106.68) (width 0.8) (layer B.Cu) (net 26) (status 20))
 (segment (start 88.9 152.4) (end 88.9 149.86) (width 0.8) (layer B.Cu) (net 7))
 (segment (start 91.44 154.94) (end 88.9 152.4) (width 0.8) (layer B.Cu) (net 7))
 (segment (start 96.52 152.4) (end 93.98 154.94) (width 0.8) (layer B.Cu) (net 7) (status 10))
 (segment (start 93.98 154.94) (end 91.44 154.94) (width 0.8) (layer B.Cu) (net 7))
 (segment (start 81.28 151.13) (end 82.55 149.86) (width 0.8) (layer B.Cu) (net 7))
 (segment (start 81.28 152.4) (end 81.28 151.13) (width 0.8) (layer B.Cu) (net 7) (status 10))
 (segment (start 82.55 149.86) (end 88.9 149.86) (width 0.8) (layer B.Cu) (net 7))
 (segment (start 95.25 113.03) (end 83.82 101.6) (width 0.8) (layer B.Cu) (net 7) (status 20))
 (segment (start 95.25 148.59) (end 95.25 113.03) (width 0.8) (layer B.Cu) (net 7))
 (segment (start 88.9 149.86) (end 93.98 149.86) (width 0.8) (layer B.Cu) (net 7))
 (segment (start 93.98 149.86) (end 95.25 148.59) (width 0.8) (layer B.Cu) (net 7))
 (segment (start 109.22 144.78) (end 109.22 149.86) (width 0.8) (layer B.Cu) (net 7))
 (segment (start 101.6 137.16) (end 109.22 144.78) (width 0.8) (layer B.Cu) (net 7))
 (segment (start 101.6 109.22) (end 101.6 137.16) (width 0.8) (layer B.Cu) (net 7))
 (segment (start 83.82 101.6) (end 93.98 101.6) (width 0.8) (layer B.Cu) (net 7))
 (segment (start 93.98 101.6) (end 101.6 109.22) (width 0.8) (layer B.Cu) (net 7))
 (segment (start 76.2 88.9) (end 73.66 88.9) (width 0.8) (layer B.Cu) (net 11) (status 20))
 (segment (start 81.28 93.98) (end 76.2 88.9) (width 0.8) (layer B.Cu) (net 11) (status 10))
 (segment (start 67.31 95.25) (end 73.66 88.9) (width 0.8) (layer B.Cu) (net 11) (status 20))
 (segment (start 63.5 95.25) (end 67.31 95.25) (width 0.8) (layer B.Cu) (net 11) (status 10))
 (segment (start 78.74 93.98) (end 81.28 96.52) (width 0.8) (layer B.Cu) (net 13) (status 20))
 (segment (start 73.66 93.98) (end 78.74 93.98) (width 0.8) (layer B.Cu) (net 13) (status 10))
 (segment (start 142.24 132.08) (end 144.78 132.08) (width 0.8) (layer B.Cu) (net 13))
 (segment (start 127 149.86) (end 127 147.32) (width 0.8) (layer B.Cu) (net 13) (status 10))
 (segment (start 127 147.32) (end 142.24 132.08) (width 0.8) (layer B.Cu) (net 13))
 (segment (start 53.34 101.6) (end 68.58 101.6) (width 0.8) (layer B.Cu) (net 13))
 (segment (start 73.66 93.98) (end 71.12 96.52) (width 0.8) (layer B.Cu) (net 13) (status 10))
 (segment (start 71.12 96.52) (end 71.12 99.06) (width 0.8) (layer B.Cu) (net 13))
 (segment (start 71.12 99.06) (end 68.58 101.6) (width 0.8) (layer B.Cu) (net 13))
 (segment (start 134.62 157.48) (end 144.78 147.32) (width 0.8) (layer B.Cu) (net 13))
 (segment (start 144.78 104.14) (end 142.24 101.6) (width 0.8) (layer B.Cu) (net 13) (status 20))
 (segment (start 144.78 147.32) (end 144.78 104.14) (width 0.8) (layer B.Cu) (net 13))
 (segment (start 63.5 89.25) (end 55.53 89.25) (width 0.8) (layer B.Cu) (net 13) (status 10))
 (segment (start 55.53 89.25) (end 53.34 91.44) (width 0.8) (layer B.Cu) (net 13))
 (segment (start 53.34 91.44) (end 53.34 144.78) (width 0.8) (layer B.Cu) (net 13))
 (segment (start 53.34 144.78) (end 50.8 147.32) (width 0.8) (layer B.Cu) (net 13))
 (segment (start 50.8 149.86) (end 58.42 157.48) (width 0.8) (layer B.Cu) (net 13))
 (segment (start 50.8 147.32) (end 50.8 149.86) (width 0.8) (layer B.Cu) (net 13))
 (segment (start 127 154.94) (end 127 157.48) (width 0.8) (layer B.Cu) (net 13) (status 10))
 (segment (start 58.42 157.48) (end 127 157.48) (width 0.8) (layer B.Cu) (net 13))
 (segment (start 127 157.48) (end 134.62 157.48) (width 0.8) (layer B.Cu) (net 13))
 (segment (start 99.06 127) (end 99.06 152.4) (width 0.8) (layer B.Cu) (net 8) (status 30))
 (segment (start 99.06 156.21) (end 59.69 156.21) (width 0.8) (layer B.Cu) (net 8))
 (segment (start 99.06 156.21) (end 99.06 152.4) (width 0.8) (layer B.Cu) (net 8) (status 20))
 (segment (start 83.82 152.4) (end 83.82 156.21) (width 0.8) (layer B.Cu) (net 8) (status 10))
 (segment (start 59.69 156.21) (end 53.34 149.86) (width 0.8) (layer B.Cu) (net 8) (status 20))
 (segment (start 115.57 156.21) (end 119.38 152.4) (width 0.8) (layer B.Cu) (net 8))
 (segment (start 111.76 156.21) (end 115.57 156.21) (width 0.8) (layer B.Cu) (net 8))
 (segment (start 96.52 91.44) (end 83.82 91.44) (width 0.8) (layer B.Cu) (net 8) (status 20))
 (segment (start 105.41 133.08001) (end 105.41 100.33) (width 0.8) (layer B.Cu) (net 8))
 (segment (start 105.41 100.33) (end 96.52 91.44) (width 0.8) (layer B.Cu) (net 8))
 (segment (start 119.38 152.4) (end 119.38 147.32) (width 0.8) (layer B.Cu) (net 8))
 (segment (start 119.38 147.32) (end 105.41 133.08001) (width 0.8) (layer B.Cu) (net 8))
 (segment (start 111.76 156.21) (end 99.06 156.21) (width 0.8) (layer B.Cu) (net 8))
 (segment (start 111.76 149.86) (end 111.76 156.21) (width 0.8) (layer B.Cu) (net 8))
 (segment (start 132.08 152.4) (end 127 152.4) (width 0.8) (layer B.Cu) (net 12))
 (segment (start 92.71 85.09) (end 80.01 85.09) (width 0.8) (layer B.Cu) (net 12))
 (segment (start 106.68 99.06) (end 92.71 85.09) (width 0.8) (layer B.Cu) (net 12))
 (segment (start 127 152.4) (end 106.68 132.08) (width 0.8) (layer B.Cu) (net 12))
 (segment (start 106.68 132.08) (end 106.68 99.06) (width 0.8) (layer B.Cu) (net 12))
 (segment (start 142.24 129.54) (end 123.19 148.59) (width 0.8) (layer B.Cu) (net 12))
 (segment (start 78.74 86.36) (end 80.01 85.09) (width 0.8) (layer B.Cu) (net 12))
 (segment (start 81.28 91.44) (end 78.74 88.9) (width 0.8) (layer B.Cu) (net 12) (status 10))
 (segment (start 78.74 88.9) (end 78.74 86.36) (width 0.8) (layer B.Cu) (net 12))
 (segment (start 142.24 129.54) (end 142.24 124.46) (width 0.8) (layer B.Cu) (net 12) (status 20))
 (segment (start 132.08 152.4) (end 134.62 149.86) (width 0.8) (layer B.Cu) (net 12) (status 20))
 (segment (start 132.08 152.4) (end 132.08 154.94) (width 0.8) (layer B.Cu) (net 12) (status 20)))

